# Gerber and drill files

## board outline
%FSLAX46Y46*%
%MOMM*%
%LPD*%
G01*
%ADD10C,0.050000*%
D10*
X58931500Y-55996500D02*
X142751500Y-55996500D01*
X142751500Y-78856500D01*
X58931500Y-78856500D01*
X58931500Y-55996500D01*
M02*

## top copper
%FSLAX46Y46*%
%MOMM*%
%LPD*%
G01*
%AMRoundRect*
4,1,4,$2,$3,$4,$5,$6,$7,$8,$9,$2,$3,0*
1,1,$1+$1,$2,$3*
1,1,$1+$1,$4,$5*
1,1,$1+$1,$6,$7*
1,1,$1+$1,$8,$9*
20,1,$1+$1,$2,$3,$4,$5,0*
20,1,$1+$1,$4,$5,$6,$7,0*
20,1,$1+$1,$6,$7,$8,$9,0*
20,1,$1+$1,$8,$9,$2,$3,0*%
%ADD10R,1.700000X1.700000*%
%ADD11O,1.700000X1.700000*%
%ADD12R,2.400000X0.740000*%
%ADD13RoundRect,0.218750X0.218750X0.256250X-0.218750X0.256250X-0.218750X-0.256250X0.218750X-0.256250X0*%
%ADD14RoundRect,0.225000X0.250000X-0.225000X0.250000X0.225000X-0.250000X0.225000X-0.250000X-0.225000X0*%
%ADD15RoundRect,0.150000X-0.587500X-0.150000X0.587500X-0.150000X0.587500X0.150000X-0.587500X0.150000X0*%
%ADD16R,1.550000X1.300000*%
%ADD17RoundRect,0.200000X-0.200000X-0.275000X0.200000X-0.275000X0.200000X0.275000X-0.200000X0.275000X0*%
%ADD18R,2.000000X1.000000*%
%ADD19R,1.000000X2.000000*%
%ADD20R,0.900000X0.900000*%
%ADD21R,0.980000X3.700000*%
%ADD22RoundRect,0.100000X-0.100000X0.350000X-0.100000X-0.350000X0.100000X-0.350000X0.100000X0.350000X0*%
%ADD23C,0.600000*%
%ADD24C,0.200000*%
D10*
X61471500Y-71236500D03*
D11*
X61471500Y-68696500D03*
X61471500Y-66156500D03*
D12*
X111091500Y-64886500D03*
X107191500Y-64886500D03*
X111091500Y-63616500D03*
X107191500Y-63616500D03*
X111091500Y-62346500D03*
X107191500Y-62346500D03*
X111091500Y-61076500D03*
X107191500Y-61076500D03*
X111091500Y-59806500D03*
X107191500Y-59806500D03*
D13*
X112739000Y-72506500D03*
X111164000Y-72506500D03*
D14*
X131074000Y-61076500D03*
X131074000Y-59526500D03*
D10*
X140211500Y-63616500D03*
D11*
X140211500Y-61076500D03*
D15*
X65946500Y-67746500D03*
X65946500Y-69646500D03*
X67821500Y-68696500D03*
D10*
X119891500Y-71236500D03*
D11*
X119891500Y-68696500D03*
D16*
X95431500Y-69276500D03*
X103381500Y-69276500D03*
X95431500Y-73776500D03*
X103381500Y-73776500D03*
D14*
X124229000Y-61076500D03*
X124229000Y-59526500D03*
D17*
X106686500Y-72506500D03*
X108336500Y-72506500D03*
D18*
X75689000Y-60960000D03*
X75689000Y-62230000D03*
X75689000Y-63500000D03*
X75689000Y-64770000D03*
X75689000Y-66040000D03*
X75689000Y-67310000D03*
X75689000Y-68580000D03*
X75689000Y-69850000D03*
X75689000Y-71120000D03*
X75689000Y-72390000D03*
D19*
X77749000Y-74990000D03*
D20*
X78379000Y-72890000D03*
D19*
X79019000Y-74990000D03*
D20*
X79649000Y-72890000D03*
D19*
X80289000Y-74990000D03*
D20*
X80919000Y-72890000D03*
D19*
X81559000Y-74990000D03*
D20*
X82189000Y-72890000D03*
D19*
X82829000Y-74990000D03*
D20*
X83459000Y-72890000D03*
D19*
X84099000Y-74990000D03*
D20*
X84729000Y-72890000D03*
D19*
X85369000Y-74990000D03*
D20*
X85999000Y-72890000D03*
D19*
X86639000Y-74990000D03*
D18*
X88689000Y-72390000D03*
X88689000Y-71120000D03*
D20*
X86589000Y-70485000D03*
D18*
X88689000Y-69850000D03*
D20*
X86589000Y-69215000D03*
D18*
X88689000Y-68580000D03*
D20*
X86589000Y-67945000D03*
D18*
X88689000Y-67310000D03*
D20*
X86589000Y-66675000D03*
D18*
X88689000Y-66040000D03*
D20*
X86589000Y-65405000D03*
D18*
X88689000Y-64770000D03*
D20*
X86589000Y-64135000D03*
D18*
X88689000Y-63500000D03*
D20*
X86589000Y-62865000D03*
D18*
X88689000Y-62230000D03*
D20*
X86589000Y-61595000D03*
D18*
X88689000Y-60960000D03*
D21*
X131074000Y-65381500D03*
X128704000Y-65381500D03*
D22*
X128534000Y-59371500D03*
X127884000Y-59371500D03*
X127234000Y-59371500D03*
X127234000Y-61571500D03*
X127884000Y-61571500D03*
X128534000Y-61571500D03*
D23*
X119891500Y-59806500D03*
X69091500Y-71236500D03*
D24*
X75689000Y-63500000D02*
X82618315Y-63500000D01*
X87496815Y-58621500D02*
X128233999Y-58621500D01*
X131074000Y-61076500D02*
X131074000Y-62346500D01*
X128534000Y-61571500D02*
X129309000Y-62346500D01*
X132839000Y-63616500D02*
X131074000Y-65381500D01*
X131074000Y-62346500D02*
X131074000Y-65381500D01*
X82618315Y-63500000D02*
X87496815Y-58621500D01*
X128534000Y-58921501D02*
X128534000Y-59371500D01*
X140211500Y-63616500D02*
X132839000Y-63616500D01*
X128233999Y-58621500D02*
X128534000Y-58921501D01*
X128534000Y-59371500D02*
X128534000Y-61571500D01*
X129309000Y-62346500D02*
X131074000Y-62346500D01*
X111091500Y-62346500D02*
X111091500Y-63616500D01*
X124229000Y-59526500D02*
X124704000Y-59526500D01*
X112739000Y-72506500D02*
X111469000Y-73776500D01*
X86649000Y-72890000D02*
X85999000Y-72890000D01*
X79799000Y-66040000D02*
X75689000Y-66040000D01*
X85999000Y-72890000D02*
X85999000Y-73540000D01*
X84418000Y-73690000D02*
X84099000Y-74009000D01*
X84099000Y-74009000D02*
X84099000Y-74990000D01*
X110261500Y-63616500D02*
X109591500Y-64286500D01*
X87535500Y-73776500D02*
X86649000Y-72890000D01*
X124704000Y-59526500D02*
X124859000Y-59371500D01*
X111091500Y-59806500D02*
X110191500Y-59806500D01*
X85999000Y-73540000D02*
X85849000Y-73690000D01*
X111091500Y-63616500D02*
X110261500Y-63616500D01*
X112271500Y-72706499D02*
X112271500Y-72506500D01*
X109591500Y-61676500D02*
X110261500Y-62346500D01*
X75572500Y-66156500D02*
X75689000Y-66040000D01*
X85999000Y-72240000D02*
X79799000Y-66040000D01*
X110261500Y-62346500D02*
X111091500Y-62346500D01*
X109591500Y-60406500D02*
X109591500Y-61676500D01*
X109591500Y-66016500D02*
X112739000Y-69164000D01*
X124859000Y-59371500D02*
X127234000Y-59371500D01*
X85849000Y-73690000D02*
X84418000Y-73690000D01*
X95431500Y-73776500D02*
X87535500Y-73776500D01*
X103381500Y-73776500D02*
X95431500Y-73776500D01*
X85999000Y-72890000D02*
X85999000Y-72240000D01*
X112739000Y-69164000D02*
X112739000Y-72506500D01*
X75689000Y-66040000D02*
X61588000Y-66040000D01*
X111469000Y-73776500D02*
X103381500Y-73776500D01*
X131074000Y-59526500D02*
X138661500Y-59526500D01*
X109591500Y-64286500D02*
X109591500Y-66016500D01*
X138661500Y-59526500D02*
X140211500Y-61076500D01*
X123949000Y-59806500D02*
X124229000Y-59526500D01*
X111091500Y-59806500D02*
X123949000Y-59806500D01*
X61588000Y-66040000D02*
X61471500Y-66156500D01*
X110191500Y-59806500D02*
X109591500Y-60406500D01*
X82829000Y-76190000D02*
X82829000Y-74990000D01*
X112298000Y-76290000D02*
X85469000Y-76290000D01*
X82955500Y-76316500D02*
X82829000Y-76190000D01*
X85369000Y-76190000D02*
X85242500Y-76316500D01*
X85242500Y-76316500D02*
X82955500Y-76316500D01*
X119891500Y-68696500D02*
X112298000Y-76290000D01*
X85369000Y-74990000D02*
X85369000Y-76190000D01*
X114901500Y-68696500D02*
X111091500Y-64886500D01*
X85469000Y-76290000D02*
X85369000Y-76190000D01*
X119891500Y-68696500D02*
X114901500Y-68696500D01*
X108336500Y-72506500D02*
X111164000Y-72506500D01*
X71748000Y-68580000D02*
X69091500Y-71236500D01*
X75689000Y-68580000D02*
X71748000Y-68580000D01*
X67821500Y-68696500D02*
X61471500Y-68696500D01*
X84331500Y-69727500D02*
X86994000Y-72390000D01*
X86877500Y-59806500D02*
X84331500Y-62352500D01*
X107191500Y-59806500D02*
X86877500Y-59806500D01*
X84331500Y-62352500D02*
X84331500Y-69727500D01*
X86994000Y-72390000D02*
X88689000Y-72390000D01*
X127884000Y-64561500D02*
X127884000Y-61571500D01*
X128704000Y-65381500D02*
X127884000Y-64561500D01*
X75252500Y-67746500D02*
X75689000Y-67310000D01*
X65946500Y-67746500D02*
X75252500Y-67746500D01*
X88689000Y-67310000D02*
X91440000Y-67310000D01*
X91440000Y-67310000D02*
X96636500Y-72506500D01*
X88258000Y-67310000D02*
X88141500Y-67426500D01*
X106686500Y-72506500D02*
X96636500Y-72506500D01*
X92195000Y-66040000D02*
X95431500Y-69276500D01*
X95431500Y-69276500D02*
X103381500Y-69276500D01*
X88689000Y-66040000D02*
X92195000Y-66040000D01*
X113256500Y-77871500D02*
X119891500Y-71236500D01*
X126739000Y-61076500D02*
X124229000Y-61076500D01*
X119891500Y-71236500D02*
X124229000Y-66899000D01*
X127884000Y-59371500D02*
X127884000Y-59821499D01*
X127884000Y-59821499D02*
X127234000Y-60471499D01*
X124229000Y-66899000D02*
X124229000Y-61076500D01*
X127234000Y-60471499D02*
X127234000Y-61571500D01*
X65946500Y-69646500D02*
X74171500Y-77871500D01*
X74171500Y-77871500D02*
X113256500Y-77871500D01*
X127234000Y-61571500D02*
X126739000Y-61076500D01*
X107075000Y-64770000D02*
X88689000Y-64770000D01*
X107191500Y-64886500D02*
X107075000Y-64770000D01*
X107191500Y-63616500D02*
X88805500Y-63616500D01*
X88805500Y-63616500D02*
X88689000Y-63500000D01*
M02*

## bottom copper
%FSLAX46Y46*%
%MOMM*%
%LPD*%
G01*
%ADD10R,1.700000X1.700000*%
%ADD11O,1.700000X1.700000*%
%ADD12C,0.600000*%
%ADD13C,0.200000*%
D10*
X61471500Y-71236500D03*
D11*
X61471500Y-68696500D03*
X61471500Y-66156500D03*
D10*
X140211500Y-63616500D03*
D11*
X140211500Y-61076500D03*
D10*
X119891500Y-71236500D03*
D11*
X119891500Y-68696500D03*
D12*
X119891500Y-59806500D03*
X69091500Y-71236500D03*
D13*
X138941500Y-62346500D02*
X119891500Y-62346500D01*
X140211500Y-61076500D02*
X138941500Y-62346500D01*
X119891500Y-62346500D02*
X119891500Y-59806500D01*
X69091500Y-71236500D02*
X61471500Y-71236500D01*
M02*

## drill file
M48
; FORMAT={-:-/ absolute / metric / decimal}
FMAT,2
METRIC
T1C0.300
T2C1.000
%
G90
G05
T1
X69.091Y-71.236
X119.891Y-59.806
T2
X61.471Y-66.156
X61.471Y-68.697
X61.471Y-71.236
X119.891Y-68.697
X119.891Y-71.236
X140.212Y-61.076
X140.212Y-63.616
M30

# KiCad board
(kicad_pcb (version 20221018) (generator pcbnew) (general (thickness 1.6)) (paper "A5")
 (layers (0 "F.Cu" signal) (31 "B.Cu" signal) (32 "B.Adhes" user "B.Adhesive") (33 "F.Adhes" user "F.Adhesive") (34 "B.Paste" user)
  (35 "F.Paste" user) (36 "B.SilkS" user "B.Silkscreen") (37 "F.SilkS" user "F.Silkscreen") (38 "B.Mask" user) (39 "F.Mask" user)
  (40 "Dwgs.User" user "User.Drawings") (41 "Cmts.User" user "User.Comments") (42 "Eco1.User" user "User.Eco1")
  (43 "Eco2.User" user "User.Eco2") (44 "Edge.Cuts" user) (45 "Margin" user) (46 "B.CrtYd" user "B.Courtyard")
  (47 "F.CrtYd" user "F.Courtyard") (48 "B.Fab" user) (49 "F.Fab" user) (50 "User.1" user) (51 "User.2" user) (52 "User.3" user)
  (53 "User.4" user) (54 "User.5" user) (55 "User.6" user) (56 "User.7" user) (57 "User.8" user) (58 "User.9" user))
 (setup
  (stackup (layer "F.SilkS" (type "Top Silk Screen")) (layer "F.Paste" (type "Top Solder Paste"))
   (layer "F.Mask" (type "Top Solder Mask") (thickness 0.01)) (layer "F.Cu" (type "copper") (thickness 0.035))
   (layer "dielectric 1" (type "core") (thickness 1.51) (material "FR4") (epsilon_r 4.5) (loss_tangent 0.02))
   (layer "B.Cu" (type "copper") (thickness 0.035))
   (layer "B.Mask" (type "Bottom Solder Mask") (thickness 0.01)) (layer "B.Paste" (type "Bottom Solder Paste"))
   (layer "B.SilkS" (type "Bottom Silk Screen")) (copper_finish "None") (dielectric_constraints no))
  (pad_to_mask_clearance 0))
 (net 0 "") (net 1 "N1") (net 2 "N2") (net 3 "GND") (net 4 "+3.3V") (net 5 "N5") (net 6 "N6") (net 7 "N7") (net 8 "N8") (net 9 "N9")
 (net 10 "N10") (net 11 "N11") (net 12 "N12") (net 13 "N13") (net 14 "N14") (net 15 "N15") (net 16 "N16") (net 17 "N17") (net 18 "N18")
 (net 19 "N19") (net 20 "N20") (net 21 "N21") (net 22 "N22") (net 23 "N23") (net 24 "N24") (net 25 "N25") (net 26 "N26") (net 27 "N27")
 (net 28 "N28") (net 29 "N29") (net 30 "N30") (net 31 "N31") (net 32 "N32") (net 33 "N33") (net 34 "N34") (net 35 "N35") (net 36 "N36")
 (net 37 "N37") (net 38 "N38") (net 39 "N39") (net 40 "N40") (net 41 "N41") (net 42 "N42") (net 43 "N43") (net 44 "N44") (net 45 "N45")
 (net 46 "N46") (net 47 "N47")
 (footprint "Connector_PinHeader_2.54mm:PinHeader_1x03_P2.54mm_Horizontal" (layer "F.Cu") (at 61.4715 71.2365 180)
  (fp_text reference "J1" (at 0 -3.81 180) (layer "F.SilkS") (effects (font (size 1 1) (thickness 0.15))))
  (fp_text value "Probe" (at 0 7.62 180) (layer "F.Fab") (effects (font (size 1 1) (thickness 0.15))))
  (pad "1" thru_hole rect (at 0 0 180) (size 1.7 1.7) (drill 1) (layers "*.Cu" "*.Mask") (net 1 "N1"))
  (pad "2" thru_hole oval (at 0 2.54 180) (size 1.7 1.7) (drill 1) (layers "*.Cu" "*.Mask") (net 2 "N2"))
  (pad "3" thru_hole oval (at 0 5.08 180) (size 1.7 1.7) (drill 1) (layers "*.Cu" "*.Mask") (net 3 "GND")))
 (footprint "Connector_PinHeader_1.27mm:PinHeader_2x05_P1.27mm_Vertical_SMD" (layer "F.Cu") (at 109.1415 62.3465 180)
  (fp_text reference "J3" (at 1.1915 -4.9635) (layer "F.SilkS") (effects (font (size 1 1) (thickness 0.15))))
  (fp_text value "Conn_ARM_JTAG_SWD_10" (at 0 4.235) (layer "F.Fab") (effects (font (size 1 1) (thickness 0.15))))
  (pad "1" smd rect (at -1.95 -2.54 180) (size 2.4 0.74) (layers "F.Cu" "F.Paste" "F.Mask") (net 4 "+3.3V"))
  (pad "2" smd rect (at 1.95 -2.54 180) (size 2.4 0.74) (layers "F.Cu" "F.Paste" "F.Mask") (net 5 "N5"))
  (pad "3" smd rect (at -1.95 -1.27 180) (size 2.4 0.74) (layers "F.Cu" "F.Paste" "F.Mask") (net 3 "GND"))
  (pad "4" smd rect (at 1.95 -1.27 180) (size 2.4 0.74) (layers "F.Cu" "F.Paste" "F.Mask") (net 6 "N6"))
  (pad "5" smd rect (at -1.95 0 180) (size 2.4 0.74) (layers "F.Cu" "F.Paste" "F.Mask") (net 3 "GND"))
  (pad "6" smd rect (at 1.95 0 180) (size 2.4 0.74) (layers "F.Cu" "F.Paste" "F.Mask") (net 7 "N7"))
  (pad "7" smd rect (at -1.95 1.27 180) (size 2.4 0.74) (layers "F.Cu" "F.Paste" "F.Mask") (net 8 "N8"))
  (pad "8" smd rect (at 1.95 1.27 180) (size 2.4 0.74) (layers "F.Cu" "F.Paste" "F.Mask") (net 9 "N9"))
  (pad "9" smd rect (at -1.95 2.54 180) (size 2.4 0.74) (layers "F.Cu" "F.Paste" "F.Mask") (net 3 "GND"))
  (pad "10" smd rect (at 1.95 2.54 180) (size 2.4 0.74) (layers "F.Cu" "F.Paste" "F.Mask") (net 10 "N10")))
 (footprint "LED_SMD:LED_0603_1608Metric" (layer "F.Cu") (at 111.9515 72.5065 180)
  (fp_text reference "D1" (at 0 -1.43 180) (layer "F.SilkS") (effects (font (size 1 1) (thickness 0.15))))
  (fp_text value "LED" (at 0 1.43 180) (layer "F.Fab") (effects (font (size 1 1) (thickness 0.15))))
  (pad "1" smd roundrect (at -0.7875 0 180) (size 0.875 0.95) (layers "F.Cu" "F.Paste" "F.Mask") (roundrect_rratio 0.25) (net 3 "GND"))
  (pad "2" smd roundrect (at 0.7875 0 180) (size 0.875 0.95) (layers "F.Cu" "F.Paste" "F.Mask") (roundrect_rratio 0.25) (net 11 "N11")))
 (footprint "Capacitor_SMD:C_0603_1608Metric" (layer "F.Cu") (at 131.074 60.3015 90)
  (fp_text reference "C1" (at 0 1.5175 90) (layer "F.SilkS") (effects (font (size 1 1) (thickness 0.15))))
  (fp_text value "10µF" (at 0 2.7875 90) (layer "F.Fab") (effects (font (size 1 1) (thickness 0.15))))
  (pad "1" smd roundrect (at -0.775 0 90) (size 0.9 0.95) (layers "F.Cu" "F.Paste" "F.Mask") (roundrect_rratio 0.25) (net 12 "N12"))
  (pad "2" smd roundrect (at 0.775 0 90) (size 0.9 0.95) (layers "F.Cu" "F.Paste" "F.Mask") (roundrect_rratio 0.25) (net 3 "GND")))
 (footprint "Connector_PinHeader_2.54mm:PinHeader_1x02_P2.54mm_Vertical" (layer "F.Cu") (at 140.2115 63.6165 180)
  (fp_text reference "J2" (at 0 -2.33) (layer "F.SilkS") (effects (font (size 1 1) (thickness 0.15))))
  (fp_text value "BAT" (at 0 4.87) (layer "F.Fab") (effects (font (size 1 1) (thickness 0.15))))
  (pad "1" thru_hole rect (at 0 0 180) (size 1.7 1.7) (drill 1) (layers "*.Cu" "*.Mask") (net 12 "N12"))
  (pad "2" thru_hole oval (at 0 2.54 180) (size 1.7 1.7) (drill 1) (layers "*.Cu" "*.Mask") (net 3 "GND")))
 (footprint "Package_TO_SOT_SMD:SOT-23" (layer "F.Cu") (at 66.884 68.6965)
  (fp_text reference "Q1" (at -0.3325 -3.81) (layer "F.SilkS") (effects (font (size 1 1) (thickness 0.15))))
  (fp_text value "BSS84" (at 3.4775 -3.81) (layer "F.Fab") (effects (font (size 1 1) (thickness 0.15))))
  (pad "1" smd roundrect (at -0.9375 -0.95) (size 1.475 0.6) (layers "F.Cu" "F.Paste" "F.Mask") (roundrect_rratio 0.25) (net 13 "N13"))
  (pad "2" smd roundrect (at -0.9375 0.95) (size 1.475 0.6) (layers "F.Cu" "F.Paste" "F.Mask") (roundrect_rratio 0.25) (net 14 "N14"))
  (pad "3" smd roundrect (at 0.9375 0) (size 1.475 0.6) (layers "F.Cu" "F.Paste" "F.Mask") (roundrect_rratio 0.25) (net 2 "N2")))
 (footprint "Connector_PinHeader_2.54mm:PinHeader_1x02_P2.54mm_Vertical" (layer "F.Cu") (at 119.8915 71.2365 180)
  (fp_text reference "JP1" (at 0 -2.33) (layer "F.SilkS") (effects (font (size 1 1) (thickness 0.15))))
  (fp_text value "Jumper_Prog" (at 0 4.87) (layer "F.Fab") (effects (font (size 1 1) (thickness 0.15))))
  (pad "1" thru_hole rect (at 0 0 180) (size 1.7 1.7) (drill 1) (layers "*.Cu" "*.Mask") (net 14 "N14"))
  (pad "2" thru_hole oval (at 0 2.54 180) (size 1.7 1.7) (drill 1) (layers "*.Cu" "*.Mask") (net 4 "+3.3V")))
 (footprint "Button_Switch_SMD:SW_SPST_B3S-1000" (layer "F.Cu") (at 99.4065 71.5265)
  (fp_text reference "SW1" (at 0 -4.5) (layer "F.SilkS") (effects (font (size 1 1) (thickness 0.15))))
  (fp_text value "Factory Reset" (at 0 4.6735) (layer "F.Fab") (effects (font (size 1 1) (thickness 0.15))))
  (pad "1" smd rect (at -3.975 -2.25) (size 1.55 1.3) (layers "F.Cu" "F.Paste" "F.Mask") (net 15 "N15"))
  (pad "1" smd rect (at 3.975 -2.25) (size 1.55 1.3) (layers "F.Cu" "F.Paste" "F.Mask") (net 15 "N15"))
  (pad "2" smd rect (at -3.975 2.25) (size 1.55 1.3) (layers "F.Cu" "F.Paste" "F.Mask") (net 3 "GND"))
  (pad "2" smd rect (at 3.975 2.25) (size 1.55 1.3) (layers "F.Cu" "F.Paste" "F.Mask") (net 3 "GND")))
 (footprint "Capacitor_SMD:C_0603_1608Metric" (layer "F.Cu") (at 124.229 60.3015 90)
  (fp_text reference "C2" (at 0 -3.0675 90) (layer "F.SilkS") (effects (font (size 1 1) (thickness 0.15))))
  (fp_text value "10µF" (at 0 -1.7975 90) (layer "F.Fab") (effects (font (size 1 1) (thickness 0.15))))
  (pad "1" smd roundrect (at -0.775 0 90) (size 0.9 0.95) (layers "F.Cu" "F.Paste" "F.Mask") (roundrect_rratio 0.25) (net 14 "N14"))
  (pad "2" smd roundrect (at 0.775 0 90) (size 0.9 0.95) (layers "F.Cu" "F.Paste" "F.Mask") (roundrect_rratio 0.25) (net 3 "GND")))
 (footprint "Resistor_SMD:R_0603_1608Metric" (layer "F.Cu") (at 107.5115 72.5065)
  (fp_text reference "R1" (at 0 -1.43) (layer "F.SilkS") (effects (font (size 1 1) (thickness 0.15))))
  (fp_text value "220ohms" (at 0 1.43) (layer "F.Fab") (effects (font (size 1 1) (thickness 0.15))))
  (pad "1" smd roundrect (at -0.825 0) (size 0.8 0.95) (layers "F.Cu" "F.Paste" "F.Mask") (roundrect_rratio 0.25) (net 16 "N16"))
  (pad "2" smd roundrect (at 0.825 0) (size 0.8 0.95) (layers "F.Cu" "F.Paste" "F.Mask") (roundrect_rratio 0.25) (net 11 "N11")))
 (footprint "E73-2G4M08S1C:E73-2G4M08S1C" (layer "F.Cu") (at 82.189 65.99)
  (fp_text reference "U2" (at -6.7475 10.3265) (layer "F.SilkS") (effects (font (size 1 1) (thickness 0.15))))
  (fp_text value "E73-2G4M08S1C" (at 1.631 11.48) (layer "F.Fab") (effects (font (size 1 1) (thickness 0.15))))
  (pad "1" smd rect (at -6.5 -5.03) (size 2 1) (layers "F.Cu" "F.Paste" "F.Mask") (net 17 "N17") (solder_mask_margin 0.102))
  (pad "2" smd rect (at -6.5 -3.76) (size 2 1) (layers "F.Cu" "F.Paste" "F.Mask") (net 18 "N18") (solder_mask_margin 0.102))
  (pad "3" smd rect (at -6.5 -2.49) (size 2 1) (layers "F.Cu" "F.Paste" "F.Mask") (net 12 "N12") (solder_mask_margin 0.102))
  (pad "4" smd rect (at -6.5 -1.22) (size 2 1) (layers "F.Cu" "F.Paste" "F.Mask") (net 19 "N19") (solder_mask_margin 0.102))
  (pad "5" smd rect (at -6.5 0.05) (size 2 1) (layers "F.Cu" "F.Paste" "F.Mask") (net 3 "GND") (solder_mask_margin 0.102))
  (pad "6" smd rect (at -6.5 1.32) (size 2 1) (layers "F.Cu" "F.Paste" "F.Mask") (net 13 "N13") (solder_mask_margin 0.102))
  (pad "7" smd rect (at -6.5 2.59) (size 2 1) (layers "F.Cu" "F.Paste" "F.Mask") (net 1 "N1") (solder_mask_margin 0.102))
  (pad "8" smd rect (at -6.5 3.86) (size 2 1) (layers "F.Cu" "F.Paste" "F.Mask") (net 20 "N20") (solder_mask_margin 0.102))
  (pad "9" smd rect (at -6.5 5.13) (size 2 1) (layers "F.Cu" "F.Paste" "F.Mask") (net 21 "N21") (solder_mask_margin 0.102))
  (pad "10" smd rect (at -6.5 6.4) (size 2 1) (layers "F.Cu" "F.Paste" "F.Mask") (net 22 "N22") (solder_mask_margin 0.102))
  (pad "11" smd rect (at -4.44 9) (size 1 2) (layers "F.Cu" "F.Paste" "F.Mask") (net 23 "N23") (solder_mask_margin 0.102))
  (pad "12" smd rect (at -3.81 6.9) (size 0.9 0.9) (layers "F.Cu" "F.Paste" "F.Mask") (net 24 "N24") (solder_mask_margin 0.102))
  (pad "13" smd rect (at -3.17 9) (size 1 2) (layers "F.Cu" "F.Paste" "F.Mask") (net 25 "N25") (solder_mask_margin 0.102))
  (pad "14" smd rect (at -2.54 6.9) (size 0.9 0.9) (layers "F.Cu" "F.Paste" "F.Mask") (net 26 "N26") (solder_mask_margin 0.102))
  (pad "15" smd rect (at -1.9 9) (size 1 2) (layers "F.Cu" "F.Paste" "F.Mask") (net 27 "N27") (solder_mask_margin 0.102))
  (pad "16" smd rect (at -1.27 6.9) (size 0.9 0.9) (layers "F.Cu" "F.Paste" "F.Mask") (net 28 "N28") (solder_mask_margin 0.102))
  (pad "17" smd rect (at -0.63 9) (size 1 2) (layers "F.Cu" "F.Paste" "F.Mask") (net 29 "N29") (solder_mask_margin 0.102))
  (pad "18" smd rect (at 0 6.9) (size 0.9 0.9) (layers "F.Cu" "F.Paste" "F.Mask") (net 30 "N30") (solder_mask_margin 0.102))
  (pad "19" smd rect (at 0.64 9) (size 1 2) (layers "F.Cu" "F.Paste" "F.Mask") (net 4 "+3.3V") (solder_mask_margin 0.102))
  (pad "20" smd rect (at 1.27 6.9) (size 0.9 0.9) (layers "F.Cu" "F.Paste" "F.Mask") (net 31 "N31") (solder_mask_margin 0.102))
  (pad "21" smd rect (at 1.91 9) (size 1 2) (layers "F.Cu" "F.Paste" "F.Mask") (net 3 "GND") (solder_mask_margin 0.102))
  (pad "22" smd rect (at 2.54 6.9) (size 0.9 0.9) (layers "F.Cu" "F.Paste" "F.Mask") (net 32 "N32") (solder_mask_margin 0.102))
  (pad "23" smd rect (at 3.18 9) (size 1 2) (layers "F.Cu" "F.Paste" "F.Mask") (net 4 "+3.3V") (solder_mask_margin 0.102))
  (pad "24" smd rect (at 3.81 6.9) (size 0.9 0.9) (layers "F.Cu" "F.Paste" "F.Mask") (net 3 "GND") (solder_mask_margin 0.102))
  (pad "25" smd rect (at 4.45 9) (size 1 2) (layers "F.Cu" "F.Paste" "F.Mask") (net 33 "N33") (solder_mask_margin 0.102))
  (pad "26" smd rect (at 6.5 6.4) (size 2 1) (layers "F.Cu" "F.Paste" "F.Mask") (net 10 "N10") (solder_mask_margin 0.102))
  (pad "27" smd rect (at 6.5 5.13) (size 2 1) (layers "F.Cu" "F.Paste" "F.Mask") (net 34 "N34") (solder_mask_margin 0.102))
  (pad "28" smd rect (at 4.4 4.495) (size 0.9 0.9) (layers "F.Cu" "F.Paste" "F.Mask") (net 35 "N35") (solder_mask_margin 0.102))
  (pad "29" smd rect (at 6.5 3.86) (size 2 1) (layers "F.Cu" "F.Paste" "F.Mask") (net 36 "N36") (solder_mask_margin 0.102))
  (pad "30" smd rect (at 4.4 3.225) (size 0.9 0.9) (layers "F.Cu" "F.Paste" "F.Mask") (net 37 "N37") (solder_mask_margin 0.102))
  (pad "31" smd rect (at 6.5 2.59) (size 2 1) (layers "F.Cu" "F.Paste" "F.Mask") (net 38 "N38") (solder_mask_margin 0.102))
  (pad "32" smd rect (at 4.4 1.955) (size 0.9 0.9) (layers "F.Cu" "F.Paste" "F.Mask") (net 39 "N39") (solder_mask_margin 0.102))
  (pad "33" smd rect (at 6.5 1.32) (size 2 1) (layers "F.Cu" "F.Paste" "F.Mask") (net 16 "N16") (solder_mask_margin 0.102))
  (pad "34" smd rect (at 4.4 0.685) (size 0.9 0.9) (layers "F.Cu" "F.Paste" "F.Mask") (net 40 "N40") (solder_mask_margin 0.102))
  (pad "35" smd rect (at 6.5 0.05) (size 2 1) (layers "F.Cu" "F.Paste" "F.Mask") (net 15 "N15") (solder_mask_margin 0.102))
  (pad "36" smd rect (at 4.4 -0.585) (size 0.9 0.9) (layers "F.Cu" "F.Paste" "F.Mask") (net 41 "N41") (solder_mask_margin 0.102))
  (pad "37" smd rect (at 6.5 -1.22) (size 2 1) (layers "F.Cu" "F.Paste" "F.Mask") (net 5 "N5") (solder_mask_margin 0.102))
  (pad "38" smd rect (at 4.4 -1.855) (size 0.9 0.9) (layers "F.Cu" "F.Paste" "F.Mask") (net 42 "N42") (solder_mask_margin 0.102))
  (pad "39" smd rect (at 6.5 -2.49) (size 2 1) (layers "F.Cu" "F.Paste" "F.Mask") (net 6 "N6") (solder_mask_margin 0.102))
  (pad "40" smd rect (at 4.4 -3.125) (size 0.9 0.9) (layers "F.Cu" "F.Paste" "F.Mask") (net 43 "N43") (solder_mask_margin 0.102))
  (pad "41" smd rect (at 6.5 -3.76) (size 2 1) (layers "F.Cu" "F.Paste" "F.Mask") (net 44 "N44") (solder_mask_margin 0.102))
  (pad "42" smd rect (at 4.4 -4.395) (size 0.9 0.9) (layers "F.Cu" "F.Paste" "F.Mask") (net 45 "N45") (solder_mask_margin 0.102))
  (pad "43" smd rect (at 6.5 -5.03) (size 2 1) (layers "F.Cu" "F.Paste" "F.Mask") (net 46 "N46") (solder_mask_margin 0.102))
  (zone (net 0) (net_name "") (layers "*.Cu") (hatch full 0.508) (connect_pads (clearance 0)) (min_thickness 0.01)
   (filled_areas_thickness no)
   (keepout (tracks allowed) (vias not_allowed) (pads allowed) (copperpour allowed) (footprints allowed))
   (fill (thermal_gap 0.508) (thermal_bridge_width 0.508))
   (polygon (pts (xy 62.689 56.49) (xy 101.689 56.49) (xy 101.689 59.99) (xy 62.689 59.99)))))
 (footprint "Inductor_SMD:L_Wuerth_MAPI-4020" (layer "F.Cu") (at 129.889 65.3815 180)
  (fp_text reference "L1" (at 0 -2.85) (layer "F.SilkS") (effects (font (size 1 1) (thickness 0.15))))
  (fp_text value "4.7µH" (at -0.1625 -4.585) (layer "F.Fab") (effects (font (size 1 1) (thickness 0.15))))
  (pad "1" smd rect (at -1.185 0 180) (size 0.98 3.7) (layers "F.Cu" "F.Paste" "F.Mask") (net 12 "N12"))
  (pad "2" smd rect (at 1.185 0 180) (size 0.98 3.7) (layers "F.Cu" "F.Paste" "F.Mask") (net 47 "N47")))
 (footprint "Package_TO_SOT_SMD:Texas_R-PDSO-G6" (layer "F.Cu") (at 127.884 60.4715 -90)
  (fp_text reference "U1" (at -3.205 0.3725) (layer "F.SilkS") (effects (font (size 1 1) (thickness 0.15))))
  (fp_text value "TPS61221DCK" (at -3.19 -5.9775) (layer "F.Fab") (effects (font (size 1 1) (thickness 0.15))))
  (pad "1" smd roundrect (at -1.1 -0.65 270) (size 0.9 0.4) (layers "F.Cu" "F.Paste" "F.Mask") (roundrect_rratio 0.25) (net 12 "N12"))
  (pad "2" smd roundrect (at -1.1 0 270) (size 0.9 0.4) (layers "F.Cu" "F.Paste" "F.Mask") (roundrect_rratio 0.25) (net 14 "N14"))
  (pad "3" smd roundrect (at -1.1 0.65 270) (size 0.9 0.4) (layers "F.Cu" "F.Paste" "F.Mask") (roundrect_rratio 0.25) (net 3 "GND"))
  (pad "4" smd roundrect (at 1.1 0.65 270) (size 0.9 0.4) (layers "F.Cu" "F.Paste" "F.Mask") (roundrect_rratio 0.25) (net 14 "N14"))
  (pad "5" smd roundrect (at 1.1 0 270) (size 0.9 0.4) (layers "F.Cu" "F.Paste" "F.Mask") (roundrect_rratio 0.25) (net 47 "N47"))
  (pad "6" smd roundrect (at 1.1 -0.65 270) (size 0.9 0.4) (layers "F.Cu" "F.Paste" "F.Mask") (roundrect_rratio 0.25) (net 12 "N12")))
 (gr_rect (start 58.9315 55.9965) (end 142.7515 78.8565) (stroke (width 0.05) (type default)) (fill none) (layer "Edge.Cuts"))
 (segment (start 75.689 63.5) (end 82.618315 63.5) (width 0.2) (layer "F.Cu") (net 12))
 (segment (start 87.496815 58.6215) (end 128.233999 58.6215) (width 0.2) (layer "F.Cu") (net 12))
 (segment (start 131.074 61.0765) (end 131.074 62.3465) (width 0.2) (layer "F.Cu") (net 12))
 (segment (start 128.534 61.5715) (end 129.309 62.3465) (width 0.2) (layer "F.Cu") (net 12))
 (segment (start 132.839 63.6165) (end 131.074 65.3815) (width 0.2) (layer "F.Cu") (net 12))
 (segment (start 131.074 62.3465) (end 131.074 65.3815) (width 0.2) (layer "F.Cu") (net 12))
 (segment (start 82.618315 63.5) (end 87.496815 58.6215) (width 0.2) (layer "F.Cu") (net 12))
 (segment (start 128.534 58.921501) (end 128.534 59.3715) (width 0.2) (layer "F.Cu") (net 12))
 (segment (start 140.2115 63.6165) (end 132.839 63.6165) (width 0.2) (layer "F.Cu") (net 12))
 (segment (start 128.233999 58.6215) (end 128.534 58.921501) (width 0.2) (layer "F.Cu") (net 12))
 (segment (start 128.534 59.3715) (end 128.534 61.5715) (width 0.2) (layer "F.Cu") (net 12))
 (segment (start 129.309 62.3465) (end 131.074 62.3465) (width 0.2) (layer "F.Cu") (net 12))
 (segment (start 111.0915 62.3465) (end 111.0915 63.6165) (width 0.2) (layer "F.Cu") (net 3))
 (segment (start 124.229 59.5265) (end 124.704 59.5265) (width 0.2) (layer "F.Cu") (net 3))
 (segment (start 112.739 72.5065) (end 111.469 73.7765) (width 0.2) (layer "F.Cu") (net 3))
 (segment (start 86.649 72.89) (end 85.999 72.89) (width 0.2) (layer "F.Cu") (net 3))
 (segment (start 79.799 66.04) (end 75.689 66.04) (width 0.2) (layer "F.Cu") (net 3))
 (segment (start 85.999 72.89) (end 85.999 73.54) (width 0.2) (layer "F.Cu") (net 3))
 (segment (start 84.418 73.69) (end 84.099 74.009) (width 0.2) (layer "F.Cu") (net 3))
 (segment (start 84.099 74.009) (end 84.099 74.99) (width 0.2) (layer "F.Cu") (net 3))
 (segment (start 110.2615 63.6165) (end 109.5915 64.2865) (width 0.2) (layer "F.Cu") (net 3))
 (segment (start 87.5355 73.7765) (end 86.649 72.89) (width 0.2) (layer "F.Cu") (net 3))
 (segment (start 124.704 59.5265) (end 124.859 59.3715) (width 0.2) (layer "F.Cu") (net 3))
 (segment (start 111.0915 59.8065) (end 110.1915 59.8065) (width 0.2) (layer "F.Cu") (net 3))
 (segment (start 85.999 73.54) (end 85.849 73.69) (width 0.2) (layer "F.Cu") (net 3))
 (segment (start 111.0915 63.6165) (end 110.2615 63.6165) (width 0.2) (layer "F.Cu") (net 3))
 (segment (start 112.2715 72.706499) (end 112.2715 72.5065) (width 0.2) (layer "F.Cu") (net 3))
 (segment (start 109.5915 61.6765) (end 110.2615 62.3465) (width 0.2) (layer "F.Cu") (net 3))
 (segment (start 75.5725 66.1565) (end 75.689 66.04) (width 0.2) (layer "F.Cu") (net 3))
 (segment (start 85.999 72.24) (end 79.799 66.04) (width 0.2) (layer "F.Cu") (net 3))
 (segment (start 110.2615 62.3465) (end 111.0915 62.3465) (width 0.2) (layer "F.Cu") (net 3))
 (segment (start 109.5915 60.4065) (end 109.5915 61.6765) (width 0.2) (layer "F.Cu") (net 3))
 (segment (start 109.5915 66.0165) (end 112.739 69.164) (width 0.2) (layer "F.Cu") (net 3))
 (segment (start 124.859 59.3715) (end 127.234 59.3715) (width 0.2) (layer "F.Cu") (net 3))
 (segment (start 85.849 73.69) (end 84.418 73.69) (width 0.2) (layer "F.Cu") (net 3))
 (segment (start 95.4315 73.7765) (end 87.5355 73.7765) (width 0.2) (layer "F.Cu") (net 3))
 (segment (start 103.3815 73.7765) (end 95.4315 73.7765) (width 0.2) (layer "F.Cu") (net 3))
 (segment (start 85.999 72.89) (end 85.999 72.24) (width 0.2) (layer "F.Cu") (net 3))
 (segment (start 112.739 69.164) (end 112.739 72.5065) (width 0.2) (layer "F.Cu") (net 3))
 (segment (start 75.689 66.04) (end 61.588 66.04) (width 0.2) (layer "F.Cu") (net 3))
 (segment (start 111.469 73.7765) (end 103.3815 73.7765) (width 0.2) (layer "F.Cu") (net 3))
 (segment (start 131.074 59.5265) (end 138.6615 59.5265) (width 0.2) (layer "F.Cu") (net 3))
 (segment (start 109.5915 64.2865) (end 109.5915 66.0165) (width 0.2) (layer "F.Cu") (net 3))
 (segment (start 138.6615 59.5265) (end 140.2115 61.0765) (width 0.2) (layer "F.Cu") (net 3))
 (segment (start 123.949 59.8065) (end 124.229 59.5265) (width 0.2) (layer "F.Cu") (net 3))
 (segment (start 111.0915 59.8065) (end 123.949 59.8065) (width 0.2) (layer "F.Cu") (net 3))
 (segment (start 61.588 66.04) (end 61.4715 66.1565) (width 0.2) (layer "F.Cu") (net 3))
 (segment (start 110.1915 59.8065) (end 109.5915 60.4065) (width 0.2) (layer "F.Cu") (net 3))
 (via (at 119.8915 59.8065) (size 0.6) (drill 0.3) (layers "F.Cu" "B.Cu") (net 3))
 (segment (start 138.9415 62.3465) (end 119.8915 62.3465) (width 0.2) (layer "B.Cu") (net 3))
 (segment (start 140.2115 61.0765) (end 138.9415 62.3465) (width 0.2) (layer "B.Cu") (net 3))
 (segment (start 119.8915 62.3465) (end 119.8915 59.8065) (width 0.2) (layer "B.Cu") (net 3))
 (segment (start 82.829 76.19) (end 82.829 74.99) (width 0.2) (layer "F.Cu") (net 4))
 (segment (start 112.298 76.29) (end 85.469 76.29) (width 0.2) (layer "F.Cu") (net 4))
 (segment (start 82.9555 76.3165) (end 82.829 76.19) (width 0.2) (layer "F.Cu") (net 4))
 (segment (start 85.369 76.19) (end 85.2425 76.3165) (width 0.2) (layer "F.Cu") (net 4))
 (segment (start 85.2425 76.3165) (end 82.9555 76.3165) (width 0.2) (layer "F.Cu") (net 4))
 (segment (start 119.8915 68.6965) (end 112.298 76.29) (width 0.2) (layer "F.Cu") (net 4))
 (segment (start 85.369 74.99) (end 85.369 76.19) (width 0.2) (layer "F.Cu") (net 4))
 (segment (start 114.9015 68.6965) (end 111.0915 64.8865) (width 0.2) (layer "F.Cu") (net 4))
 (segment (start 85.469 76.29) (end 85.369 76.19) (width 0.2) (layer "F.Cu") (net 4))
 (segment (start 119.8915 68.6965) (end 114.9015 68.6965) (width 0.2) (layer "F.Cu") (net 4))
 (segment (start 108.3365 72.5065) (end 111.164 72.5065) (width 0.2) (layer "F.Cu") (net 11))
 (segment (start 71.748 68.58) (end 69.0915 71.2365) (width 0.2) (layer "F.Cu") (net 1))
 (segment (start 75.689 68.58) (end 71.748 68.58) (width 0.2) (layer "F.Cu") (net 1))
 (via (at 69.0915 71.2365) (size 0.6) (drill 0.3) (layers "F.Cu" "B.Cu") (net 1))
 (segment (start 69.0915 71.2365) (end 61.4715 71.2365) (width 0.2) (layer "B.Cu") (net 1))
 (segment (start 67.8215 68.6965) (end 61.4715 68.6965) (width 0.2) (layer "F.Cu") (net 2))
 (segment (start 84.3315 69.7275) (end 86.994 72.39) (width 0.2) (layer "F.Cu") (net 10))
 (segment (start 86.8775 59.8065) (end 84.3315 62.3525) (width 0.2) (layer "F.Cu") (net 10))
 (segment (start 107.1915 59.8065) (end 86.8775 59.8065) (width 0.2) (layer "F.Cu") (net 10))
 (segment (start 84.3315 62.3525) (end 84.3315 69.7275) (width 0.2) (layer "F.Cu") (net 10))
 (segment (start 86.994 72.39) (end 88.689 72.39) (width 0.2) (layer "F.Cu") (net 10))
 (segment (start 127.884 64.5615) (end 127.884 61.5715) (width 0.2) (layer "F.Cu") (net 47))
 (segment (start 128.704 65.3815) (end 127.884 64.5615) (width 0.2) (layer "F.Cu") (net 47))
 (segment (start 75.2525 67.7465) (end 75.689 67.31) (width 0.2) (layer "F.Cu") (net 13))
 (segment (start 65.9465 67.7465) (end 75.2525 67.7465) (width 0.2) (layer "F.Cu") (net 13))
 (segment (start 88.689 67.31) (end 91.44 67.31) (width 0.2) (layer "F.Cu") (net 16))
 (segment (start 91.44 67.31) (end 96.6365 72.5065) (width 0.2) (layer "F.Cu") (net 16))
 (segment (start 88.258 67.31) (end 88.1415 67.4265) (width 0.2) (layer "F.Cu") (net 16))
 (segment (start 106.6865 72.5065) (end 96.6365 72.5065) (width 0.2) (layer "F.Cu") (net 16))
 (segment (start 92.195 66.04) (end 95.4315 69.2765) (width 0.2) (layer "F.Cu") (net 15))
 (segment (start 95.4315 69.2765) (end 103.3815 69.2765) (width 0.2) (layer "F.Cu") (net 15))
 (segment (start 88.689 66.04) (end 92.195 66.04) (width 0.2) (layer "F.Cu") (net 15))
 (segment (start 113.2565 77.8715) (end 119.8915 71.2365) (width 0.2) (layer "F.Cu") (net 14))
 (segment (start 126.739 61.0765) (end 124.229 61.0765) (width 0.2) (layer "F.Cu") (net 14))
 (segment (start 119.8915 71.2365) (end 124.229 66.899) (width 0.2) (layer "F.Cu") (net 14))
 (segment (start 127.884 59.3715) (end 127.884 59.821499) (width 0.2) (layer "F.Cu") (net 14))
 (segment (start 127.884 59.821499) (end 127.234 60.471499) (width 0.2) (layer "F.Cu") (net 14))
 (segment (start 124.229 66.899) (end 124.229 61.0765) (width 0.2) (layer "F.Cu") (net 14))
 (segment (start 127.234 60.471499) (end 127.234 61.5715) (width 0.2) (layer "F.Cu") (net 14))
 (segment (start 65.9465 69.6465) (end 74.1715 77.8715) (width 0.2) (layer "F.Cu") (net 14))
 (segment (start 74.1715 77.8715) (end 113.2565 77.8715) (width 0.2) (layer "F.Cu") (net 14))
 (segment (start 127.234 61.5715) (end 126.739 61.0765) (width 0.2) (layer "F.Cu") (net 14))
 (segment (start 107.075 64.77) (end 88.689 64.77) (width 0.2) (layer "F.Cu") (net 5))
 (segment (start 107.1915 64.8865) (end 107.075 64.77) (width 0.2) (layer "F.Cu") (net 5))
 (segment (start 107.1915 63.6165) (end 88.8055 63.6165) (width 0.2) (layer "F.Cu") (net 6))
 (segment (start 88.8055 63.6165) (end 88.689 63.5) (width 0.2) (layer "F.Cu") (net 6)))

